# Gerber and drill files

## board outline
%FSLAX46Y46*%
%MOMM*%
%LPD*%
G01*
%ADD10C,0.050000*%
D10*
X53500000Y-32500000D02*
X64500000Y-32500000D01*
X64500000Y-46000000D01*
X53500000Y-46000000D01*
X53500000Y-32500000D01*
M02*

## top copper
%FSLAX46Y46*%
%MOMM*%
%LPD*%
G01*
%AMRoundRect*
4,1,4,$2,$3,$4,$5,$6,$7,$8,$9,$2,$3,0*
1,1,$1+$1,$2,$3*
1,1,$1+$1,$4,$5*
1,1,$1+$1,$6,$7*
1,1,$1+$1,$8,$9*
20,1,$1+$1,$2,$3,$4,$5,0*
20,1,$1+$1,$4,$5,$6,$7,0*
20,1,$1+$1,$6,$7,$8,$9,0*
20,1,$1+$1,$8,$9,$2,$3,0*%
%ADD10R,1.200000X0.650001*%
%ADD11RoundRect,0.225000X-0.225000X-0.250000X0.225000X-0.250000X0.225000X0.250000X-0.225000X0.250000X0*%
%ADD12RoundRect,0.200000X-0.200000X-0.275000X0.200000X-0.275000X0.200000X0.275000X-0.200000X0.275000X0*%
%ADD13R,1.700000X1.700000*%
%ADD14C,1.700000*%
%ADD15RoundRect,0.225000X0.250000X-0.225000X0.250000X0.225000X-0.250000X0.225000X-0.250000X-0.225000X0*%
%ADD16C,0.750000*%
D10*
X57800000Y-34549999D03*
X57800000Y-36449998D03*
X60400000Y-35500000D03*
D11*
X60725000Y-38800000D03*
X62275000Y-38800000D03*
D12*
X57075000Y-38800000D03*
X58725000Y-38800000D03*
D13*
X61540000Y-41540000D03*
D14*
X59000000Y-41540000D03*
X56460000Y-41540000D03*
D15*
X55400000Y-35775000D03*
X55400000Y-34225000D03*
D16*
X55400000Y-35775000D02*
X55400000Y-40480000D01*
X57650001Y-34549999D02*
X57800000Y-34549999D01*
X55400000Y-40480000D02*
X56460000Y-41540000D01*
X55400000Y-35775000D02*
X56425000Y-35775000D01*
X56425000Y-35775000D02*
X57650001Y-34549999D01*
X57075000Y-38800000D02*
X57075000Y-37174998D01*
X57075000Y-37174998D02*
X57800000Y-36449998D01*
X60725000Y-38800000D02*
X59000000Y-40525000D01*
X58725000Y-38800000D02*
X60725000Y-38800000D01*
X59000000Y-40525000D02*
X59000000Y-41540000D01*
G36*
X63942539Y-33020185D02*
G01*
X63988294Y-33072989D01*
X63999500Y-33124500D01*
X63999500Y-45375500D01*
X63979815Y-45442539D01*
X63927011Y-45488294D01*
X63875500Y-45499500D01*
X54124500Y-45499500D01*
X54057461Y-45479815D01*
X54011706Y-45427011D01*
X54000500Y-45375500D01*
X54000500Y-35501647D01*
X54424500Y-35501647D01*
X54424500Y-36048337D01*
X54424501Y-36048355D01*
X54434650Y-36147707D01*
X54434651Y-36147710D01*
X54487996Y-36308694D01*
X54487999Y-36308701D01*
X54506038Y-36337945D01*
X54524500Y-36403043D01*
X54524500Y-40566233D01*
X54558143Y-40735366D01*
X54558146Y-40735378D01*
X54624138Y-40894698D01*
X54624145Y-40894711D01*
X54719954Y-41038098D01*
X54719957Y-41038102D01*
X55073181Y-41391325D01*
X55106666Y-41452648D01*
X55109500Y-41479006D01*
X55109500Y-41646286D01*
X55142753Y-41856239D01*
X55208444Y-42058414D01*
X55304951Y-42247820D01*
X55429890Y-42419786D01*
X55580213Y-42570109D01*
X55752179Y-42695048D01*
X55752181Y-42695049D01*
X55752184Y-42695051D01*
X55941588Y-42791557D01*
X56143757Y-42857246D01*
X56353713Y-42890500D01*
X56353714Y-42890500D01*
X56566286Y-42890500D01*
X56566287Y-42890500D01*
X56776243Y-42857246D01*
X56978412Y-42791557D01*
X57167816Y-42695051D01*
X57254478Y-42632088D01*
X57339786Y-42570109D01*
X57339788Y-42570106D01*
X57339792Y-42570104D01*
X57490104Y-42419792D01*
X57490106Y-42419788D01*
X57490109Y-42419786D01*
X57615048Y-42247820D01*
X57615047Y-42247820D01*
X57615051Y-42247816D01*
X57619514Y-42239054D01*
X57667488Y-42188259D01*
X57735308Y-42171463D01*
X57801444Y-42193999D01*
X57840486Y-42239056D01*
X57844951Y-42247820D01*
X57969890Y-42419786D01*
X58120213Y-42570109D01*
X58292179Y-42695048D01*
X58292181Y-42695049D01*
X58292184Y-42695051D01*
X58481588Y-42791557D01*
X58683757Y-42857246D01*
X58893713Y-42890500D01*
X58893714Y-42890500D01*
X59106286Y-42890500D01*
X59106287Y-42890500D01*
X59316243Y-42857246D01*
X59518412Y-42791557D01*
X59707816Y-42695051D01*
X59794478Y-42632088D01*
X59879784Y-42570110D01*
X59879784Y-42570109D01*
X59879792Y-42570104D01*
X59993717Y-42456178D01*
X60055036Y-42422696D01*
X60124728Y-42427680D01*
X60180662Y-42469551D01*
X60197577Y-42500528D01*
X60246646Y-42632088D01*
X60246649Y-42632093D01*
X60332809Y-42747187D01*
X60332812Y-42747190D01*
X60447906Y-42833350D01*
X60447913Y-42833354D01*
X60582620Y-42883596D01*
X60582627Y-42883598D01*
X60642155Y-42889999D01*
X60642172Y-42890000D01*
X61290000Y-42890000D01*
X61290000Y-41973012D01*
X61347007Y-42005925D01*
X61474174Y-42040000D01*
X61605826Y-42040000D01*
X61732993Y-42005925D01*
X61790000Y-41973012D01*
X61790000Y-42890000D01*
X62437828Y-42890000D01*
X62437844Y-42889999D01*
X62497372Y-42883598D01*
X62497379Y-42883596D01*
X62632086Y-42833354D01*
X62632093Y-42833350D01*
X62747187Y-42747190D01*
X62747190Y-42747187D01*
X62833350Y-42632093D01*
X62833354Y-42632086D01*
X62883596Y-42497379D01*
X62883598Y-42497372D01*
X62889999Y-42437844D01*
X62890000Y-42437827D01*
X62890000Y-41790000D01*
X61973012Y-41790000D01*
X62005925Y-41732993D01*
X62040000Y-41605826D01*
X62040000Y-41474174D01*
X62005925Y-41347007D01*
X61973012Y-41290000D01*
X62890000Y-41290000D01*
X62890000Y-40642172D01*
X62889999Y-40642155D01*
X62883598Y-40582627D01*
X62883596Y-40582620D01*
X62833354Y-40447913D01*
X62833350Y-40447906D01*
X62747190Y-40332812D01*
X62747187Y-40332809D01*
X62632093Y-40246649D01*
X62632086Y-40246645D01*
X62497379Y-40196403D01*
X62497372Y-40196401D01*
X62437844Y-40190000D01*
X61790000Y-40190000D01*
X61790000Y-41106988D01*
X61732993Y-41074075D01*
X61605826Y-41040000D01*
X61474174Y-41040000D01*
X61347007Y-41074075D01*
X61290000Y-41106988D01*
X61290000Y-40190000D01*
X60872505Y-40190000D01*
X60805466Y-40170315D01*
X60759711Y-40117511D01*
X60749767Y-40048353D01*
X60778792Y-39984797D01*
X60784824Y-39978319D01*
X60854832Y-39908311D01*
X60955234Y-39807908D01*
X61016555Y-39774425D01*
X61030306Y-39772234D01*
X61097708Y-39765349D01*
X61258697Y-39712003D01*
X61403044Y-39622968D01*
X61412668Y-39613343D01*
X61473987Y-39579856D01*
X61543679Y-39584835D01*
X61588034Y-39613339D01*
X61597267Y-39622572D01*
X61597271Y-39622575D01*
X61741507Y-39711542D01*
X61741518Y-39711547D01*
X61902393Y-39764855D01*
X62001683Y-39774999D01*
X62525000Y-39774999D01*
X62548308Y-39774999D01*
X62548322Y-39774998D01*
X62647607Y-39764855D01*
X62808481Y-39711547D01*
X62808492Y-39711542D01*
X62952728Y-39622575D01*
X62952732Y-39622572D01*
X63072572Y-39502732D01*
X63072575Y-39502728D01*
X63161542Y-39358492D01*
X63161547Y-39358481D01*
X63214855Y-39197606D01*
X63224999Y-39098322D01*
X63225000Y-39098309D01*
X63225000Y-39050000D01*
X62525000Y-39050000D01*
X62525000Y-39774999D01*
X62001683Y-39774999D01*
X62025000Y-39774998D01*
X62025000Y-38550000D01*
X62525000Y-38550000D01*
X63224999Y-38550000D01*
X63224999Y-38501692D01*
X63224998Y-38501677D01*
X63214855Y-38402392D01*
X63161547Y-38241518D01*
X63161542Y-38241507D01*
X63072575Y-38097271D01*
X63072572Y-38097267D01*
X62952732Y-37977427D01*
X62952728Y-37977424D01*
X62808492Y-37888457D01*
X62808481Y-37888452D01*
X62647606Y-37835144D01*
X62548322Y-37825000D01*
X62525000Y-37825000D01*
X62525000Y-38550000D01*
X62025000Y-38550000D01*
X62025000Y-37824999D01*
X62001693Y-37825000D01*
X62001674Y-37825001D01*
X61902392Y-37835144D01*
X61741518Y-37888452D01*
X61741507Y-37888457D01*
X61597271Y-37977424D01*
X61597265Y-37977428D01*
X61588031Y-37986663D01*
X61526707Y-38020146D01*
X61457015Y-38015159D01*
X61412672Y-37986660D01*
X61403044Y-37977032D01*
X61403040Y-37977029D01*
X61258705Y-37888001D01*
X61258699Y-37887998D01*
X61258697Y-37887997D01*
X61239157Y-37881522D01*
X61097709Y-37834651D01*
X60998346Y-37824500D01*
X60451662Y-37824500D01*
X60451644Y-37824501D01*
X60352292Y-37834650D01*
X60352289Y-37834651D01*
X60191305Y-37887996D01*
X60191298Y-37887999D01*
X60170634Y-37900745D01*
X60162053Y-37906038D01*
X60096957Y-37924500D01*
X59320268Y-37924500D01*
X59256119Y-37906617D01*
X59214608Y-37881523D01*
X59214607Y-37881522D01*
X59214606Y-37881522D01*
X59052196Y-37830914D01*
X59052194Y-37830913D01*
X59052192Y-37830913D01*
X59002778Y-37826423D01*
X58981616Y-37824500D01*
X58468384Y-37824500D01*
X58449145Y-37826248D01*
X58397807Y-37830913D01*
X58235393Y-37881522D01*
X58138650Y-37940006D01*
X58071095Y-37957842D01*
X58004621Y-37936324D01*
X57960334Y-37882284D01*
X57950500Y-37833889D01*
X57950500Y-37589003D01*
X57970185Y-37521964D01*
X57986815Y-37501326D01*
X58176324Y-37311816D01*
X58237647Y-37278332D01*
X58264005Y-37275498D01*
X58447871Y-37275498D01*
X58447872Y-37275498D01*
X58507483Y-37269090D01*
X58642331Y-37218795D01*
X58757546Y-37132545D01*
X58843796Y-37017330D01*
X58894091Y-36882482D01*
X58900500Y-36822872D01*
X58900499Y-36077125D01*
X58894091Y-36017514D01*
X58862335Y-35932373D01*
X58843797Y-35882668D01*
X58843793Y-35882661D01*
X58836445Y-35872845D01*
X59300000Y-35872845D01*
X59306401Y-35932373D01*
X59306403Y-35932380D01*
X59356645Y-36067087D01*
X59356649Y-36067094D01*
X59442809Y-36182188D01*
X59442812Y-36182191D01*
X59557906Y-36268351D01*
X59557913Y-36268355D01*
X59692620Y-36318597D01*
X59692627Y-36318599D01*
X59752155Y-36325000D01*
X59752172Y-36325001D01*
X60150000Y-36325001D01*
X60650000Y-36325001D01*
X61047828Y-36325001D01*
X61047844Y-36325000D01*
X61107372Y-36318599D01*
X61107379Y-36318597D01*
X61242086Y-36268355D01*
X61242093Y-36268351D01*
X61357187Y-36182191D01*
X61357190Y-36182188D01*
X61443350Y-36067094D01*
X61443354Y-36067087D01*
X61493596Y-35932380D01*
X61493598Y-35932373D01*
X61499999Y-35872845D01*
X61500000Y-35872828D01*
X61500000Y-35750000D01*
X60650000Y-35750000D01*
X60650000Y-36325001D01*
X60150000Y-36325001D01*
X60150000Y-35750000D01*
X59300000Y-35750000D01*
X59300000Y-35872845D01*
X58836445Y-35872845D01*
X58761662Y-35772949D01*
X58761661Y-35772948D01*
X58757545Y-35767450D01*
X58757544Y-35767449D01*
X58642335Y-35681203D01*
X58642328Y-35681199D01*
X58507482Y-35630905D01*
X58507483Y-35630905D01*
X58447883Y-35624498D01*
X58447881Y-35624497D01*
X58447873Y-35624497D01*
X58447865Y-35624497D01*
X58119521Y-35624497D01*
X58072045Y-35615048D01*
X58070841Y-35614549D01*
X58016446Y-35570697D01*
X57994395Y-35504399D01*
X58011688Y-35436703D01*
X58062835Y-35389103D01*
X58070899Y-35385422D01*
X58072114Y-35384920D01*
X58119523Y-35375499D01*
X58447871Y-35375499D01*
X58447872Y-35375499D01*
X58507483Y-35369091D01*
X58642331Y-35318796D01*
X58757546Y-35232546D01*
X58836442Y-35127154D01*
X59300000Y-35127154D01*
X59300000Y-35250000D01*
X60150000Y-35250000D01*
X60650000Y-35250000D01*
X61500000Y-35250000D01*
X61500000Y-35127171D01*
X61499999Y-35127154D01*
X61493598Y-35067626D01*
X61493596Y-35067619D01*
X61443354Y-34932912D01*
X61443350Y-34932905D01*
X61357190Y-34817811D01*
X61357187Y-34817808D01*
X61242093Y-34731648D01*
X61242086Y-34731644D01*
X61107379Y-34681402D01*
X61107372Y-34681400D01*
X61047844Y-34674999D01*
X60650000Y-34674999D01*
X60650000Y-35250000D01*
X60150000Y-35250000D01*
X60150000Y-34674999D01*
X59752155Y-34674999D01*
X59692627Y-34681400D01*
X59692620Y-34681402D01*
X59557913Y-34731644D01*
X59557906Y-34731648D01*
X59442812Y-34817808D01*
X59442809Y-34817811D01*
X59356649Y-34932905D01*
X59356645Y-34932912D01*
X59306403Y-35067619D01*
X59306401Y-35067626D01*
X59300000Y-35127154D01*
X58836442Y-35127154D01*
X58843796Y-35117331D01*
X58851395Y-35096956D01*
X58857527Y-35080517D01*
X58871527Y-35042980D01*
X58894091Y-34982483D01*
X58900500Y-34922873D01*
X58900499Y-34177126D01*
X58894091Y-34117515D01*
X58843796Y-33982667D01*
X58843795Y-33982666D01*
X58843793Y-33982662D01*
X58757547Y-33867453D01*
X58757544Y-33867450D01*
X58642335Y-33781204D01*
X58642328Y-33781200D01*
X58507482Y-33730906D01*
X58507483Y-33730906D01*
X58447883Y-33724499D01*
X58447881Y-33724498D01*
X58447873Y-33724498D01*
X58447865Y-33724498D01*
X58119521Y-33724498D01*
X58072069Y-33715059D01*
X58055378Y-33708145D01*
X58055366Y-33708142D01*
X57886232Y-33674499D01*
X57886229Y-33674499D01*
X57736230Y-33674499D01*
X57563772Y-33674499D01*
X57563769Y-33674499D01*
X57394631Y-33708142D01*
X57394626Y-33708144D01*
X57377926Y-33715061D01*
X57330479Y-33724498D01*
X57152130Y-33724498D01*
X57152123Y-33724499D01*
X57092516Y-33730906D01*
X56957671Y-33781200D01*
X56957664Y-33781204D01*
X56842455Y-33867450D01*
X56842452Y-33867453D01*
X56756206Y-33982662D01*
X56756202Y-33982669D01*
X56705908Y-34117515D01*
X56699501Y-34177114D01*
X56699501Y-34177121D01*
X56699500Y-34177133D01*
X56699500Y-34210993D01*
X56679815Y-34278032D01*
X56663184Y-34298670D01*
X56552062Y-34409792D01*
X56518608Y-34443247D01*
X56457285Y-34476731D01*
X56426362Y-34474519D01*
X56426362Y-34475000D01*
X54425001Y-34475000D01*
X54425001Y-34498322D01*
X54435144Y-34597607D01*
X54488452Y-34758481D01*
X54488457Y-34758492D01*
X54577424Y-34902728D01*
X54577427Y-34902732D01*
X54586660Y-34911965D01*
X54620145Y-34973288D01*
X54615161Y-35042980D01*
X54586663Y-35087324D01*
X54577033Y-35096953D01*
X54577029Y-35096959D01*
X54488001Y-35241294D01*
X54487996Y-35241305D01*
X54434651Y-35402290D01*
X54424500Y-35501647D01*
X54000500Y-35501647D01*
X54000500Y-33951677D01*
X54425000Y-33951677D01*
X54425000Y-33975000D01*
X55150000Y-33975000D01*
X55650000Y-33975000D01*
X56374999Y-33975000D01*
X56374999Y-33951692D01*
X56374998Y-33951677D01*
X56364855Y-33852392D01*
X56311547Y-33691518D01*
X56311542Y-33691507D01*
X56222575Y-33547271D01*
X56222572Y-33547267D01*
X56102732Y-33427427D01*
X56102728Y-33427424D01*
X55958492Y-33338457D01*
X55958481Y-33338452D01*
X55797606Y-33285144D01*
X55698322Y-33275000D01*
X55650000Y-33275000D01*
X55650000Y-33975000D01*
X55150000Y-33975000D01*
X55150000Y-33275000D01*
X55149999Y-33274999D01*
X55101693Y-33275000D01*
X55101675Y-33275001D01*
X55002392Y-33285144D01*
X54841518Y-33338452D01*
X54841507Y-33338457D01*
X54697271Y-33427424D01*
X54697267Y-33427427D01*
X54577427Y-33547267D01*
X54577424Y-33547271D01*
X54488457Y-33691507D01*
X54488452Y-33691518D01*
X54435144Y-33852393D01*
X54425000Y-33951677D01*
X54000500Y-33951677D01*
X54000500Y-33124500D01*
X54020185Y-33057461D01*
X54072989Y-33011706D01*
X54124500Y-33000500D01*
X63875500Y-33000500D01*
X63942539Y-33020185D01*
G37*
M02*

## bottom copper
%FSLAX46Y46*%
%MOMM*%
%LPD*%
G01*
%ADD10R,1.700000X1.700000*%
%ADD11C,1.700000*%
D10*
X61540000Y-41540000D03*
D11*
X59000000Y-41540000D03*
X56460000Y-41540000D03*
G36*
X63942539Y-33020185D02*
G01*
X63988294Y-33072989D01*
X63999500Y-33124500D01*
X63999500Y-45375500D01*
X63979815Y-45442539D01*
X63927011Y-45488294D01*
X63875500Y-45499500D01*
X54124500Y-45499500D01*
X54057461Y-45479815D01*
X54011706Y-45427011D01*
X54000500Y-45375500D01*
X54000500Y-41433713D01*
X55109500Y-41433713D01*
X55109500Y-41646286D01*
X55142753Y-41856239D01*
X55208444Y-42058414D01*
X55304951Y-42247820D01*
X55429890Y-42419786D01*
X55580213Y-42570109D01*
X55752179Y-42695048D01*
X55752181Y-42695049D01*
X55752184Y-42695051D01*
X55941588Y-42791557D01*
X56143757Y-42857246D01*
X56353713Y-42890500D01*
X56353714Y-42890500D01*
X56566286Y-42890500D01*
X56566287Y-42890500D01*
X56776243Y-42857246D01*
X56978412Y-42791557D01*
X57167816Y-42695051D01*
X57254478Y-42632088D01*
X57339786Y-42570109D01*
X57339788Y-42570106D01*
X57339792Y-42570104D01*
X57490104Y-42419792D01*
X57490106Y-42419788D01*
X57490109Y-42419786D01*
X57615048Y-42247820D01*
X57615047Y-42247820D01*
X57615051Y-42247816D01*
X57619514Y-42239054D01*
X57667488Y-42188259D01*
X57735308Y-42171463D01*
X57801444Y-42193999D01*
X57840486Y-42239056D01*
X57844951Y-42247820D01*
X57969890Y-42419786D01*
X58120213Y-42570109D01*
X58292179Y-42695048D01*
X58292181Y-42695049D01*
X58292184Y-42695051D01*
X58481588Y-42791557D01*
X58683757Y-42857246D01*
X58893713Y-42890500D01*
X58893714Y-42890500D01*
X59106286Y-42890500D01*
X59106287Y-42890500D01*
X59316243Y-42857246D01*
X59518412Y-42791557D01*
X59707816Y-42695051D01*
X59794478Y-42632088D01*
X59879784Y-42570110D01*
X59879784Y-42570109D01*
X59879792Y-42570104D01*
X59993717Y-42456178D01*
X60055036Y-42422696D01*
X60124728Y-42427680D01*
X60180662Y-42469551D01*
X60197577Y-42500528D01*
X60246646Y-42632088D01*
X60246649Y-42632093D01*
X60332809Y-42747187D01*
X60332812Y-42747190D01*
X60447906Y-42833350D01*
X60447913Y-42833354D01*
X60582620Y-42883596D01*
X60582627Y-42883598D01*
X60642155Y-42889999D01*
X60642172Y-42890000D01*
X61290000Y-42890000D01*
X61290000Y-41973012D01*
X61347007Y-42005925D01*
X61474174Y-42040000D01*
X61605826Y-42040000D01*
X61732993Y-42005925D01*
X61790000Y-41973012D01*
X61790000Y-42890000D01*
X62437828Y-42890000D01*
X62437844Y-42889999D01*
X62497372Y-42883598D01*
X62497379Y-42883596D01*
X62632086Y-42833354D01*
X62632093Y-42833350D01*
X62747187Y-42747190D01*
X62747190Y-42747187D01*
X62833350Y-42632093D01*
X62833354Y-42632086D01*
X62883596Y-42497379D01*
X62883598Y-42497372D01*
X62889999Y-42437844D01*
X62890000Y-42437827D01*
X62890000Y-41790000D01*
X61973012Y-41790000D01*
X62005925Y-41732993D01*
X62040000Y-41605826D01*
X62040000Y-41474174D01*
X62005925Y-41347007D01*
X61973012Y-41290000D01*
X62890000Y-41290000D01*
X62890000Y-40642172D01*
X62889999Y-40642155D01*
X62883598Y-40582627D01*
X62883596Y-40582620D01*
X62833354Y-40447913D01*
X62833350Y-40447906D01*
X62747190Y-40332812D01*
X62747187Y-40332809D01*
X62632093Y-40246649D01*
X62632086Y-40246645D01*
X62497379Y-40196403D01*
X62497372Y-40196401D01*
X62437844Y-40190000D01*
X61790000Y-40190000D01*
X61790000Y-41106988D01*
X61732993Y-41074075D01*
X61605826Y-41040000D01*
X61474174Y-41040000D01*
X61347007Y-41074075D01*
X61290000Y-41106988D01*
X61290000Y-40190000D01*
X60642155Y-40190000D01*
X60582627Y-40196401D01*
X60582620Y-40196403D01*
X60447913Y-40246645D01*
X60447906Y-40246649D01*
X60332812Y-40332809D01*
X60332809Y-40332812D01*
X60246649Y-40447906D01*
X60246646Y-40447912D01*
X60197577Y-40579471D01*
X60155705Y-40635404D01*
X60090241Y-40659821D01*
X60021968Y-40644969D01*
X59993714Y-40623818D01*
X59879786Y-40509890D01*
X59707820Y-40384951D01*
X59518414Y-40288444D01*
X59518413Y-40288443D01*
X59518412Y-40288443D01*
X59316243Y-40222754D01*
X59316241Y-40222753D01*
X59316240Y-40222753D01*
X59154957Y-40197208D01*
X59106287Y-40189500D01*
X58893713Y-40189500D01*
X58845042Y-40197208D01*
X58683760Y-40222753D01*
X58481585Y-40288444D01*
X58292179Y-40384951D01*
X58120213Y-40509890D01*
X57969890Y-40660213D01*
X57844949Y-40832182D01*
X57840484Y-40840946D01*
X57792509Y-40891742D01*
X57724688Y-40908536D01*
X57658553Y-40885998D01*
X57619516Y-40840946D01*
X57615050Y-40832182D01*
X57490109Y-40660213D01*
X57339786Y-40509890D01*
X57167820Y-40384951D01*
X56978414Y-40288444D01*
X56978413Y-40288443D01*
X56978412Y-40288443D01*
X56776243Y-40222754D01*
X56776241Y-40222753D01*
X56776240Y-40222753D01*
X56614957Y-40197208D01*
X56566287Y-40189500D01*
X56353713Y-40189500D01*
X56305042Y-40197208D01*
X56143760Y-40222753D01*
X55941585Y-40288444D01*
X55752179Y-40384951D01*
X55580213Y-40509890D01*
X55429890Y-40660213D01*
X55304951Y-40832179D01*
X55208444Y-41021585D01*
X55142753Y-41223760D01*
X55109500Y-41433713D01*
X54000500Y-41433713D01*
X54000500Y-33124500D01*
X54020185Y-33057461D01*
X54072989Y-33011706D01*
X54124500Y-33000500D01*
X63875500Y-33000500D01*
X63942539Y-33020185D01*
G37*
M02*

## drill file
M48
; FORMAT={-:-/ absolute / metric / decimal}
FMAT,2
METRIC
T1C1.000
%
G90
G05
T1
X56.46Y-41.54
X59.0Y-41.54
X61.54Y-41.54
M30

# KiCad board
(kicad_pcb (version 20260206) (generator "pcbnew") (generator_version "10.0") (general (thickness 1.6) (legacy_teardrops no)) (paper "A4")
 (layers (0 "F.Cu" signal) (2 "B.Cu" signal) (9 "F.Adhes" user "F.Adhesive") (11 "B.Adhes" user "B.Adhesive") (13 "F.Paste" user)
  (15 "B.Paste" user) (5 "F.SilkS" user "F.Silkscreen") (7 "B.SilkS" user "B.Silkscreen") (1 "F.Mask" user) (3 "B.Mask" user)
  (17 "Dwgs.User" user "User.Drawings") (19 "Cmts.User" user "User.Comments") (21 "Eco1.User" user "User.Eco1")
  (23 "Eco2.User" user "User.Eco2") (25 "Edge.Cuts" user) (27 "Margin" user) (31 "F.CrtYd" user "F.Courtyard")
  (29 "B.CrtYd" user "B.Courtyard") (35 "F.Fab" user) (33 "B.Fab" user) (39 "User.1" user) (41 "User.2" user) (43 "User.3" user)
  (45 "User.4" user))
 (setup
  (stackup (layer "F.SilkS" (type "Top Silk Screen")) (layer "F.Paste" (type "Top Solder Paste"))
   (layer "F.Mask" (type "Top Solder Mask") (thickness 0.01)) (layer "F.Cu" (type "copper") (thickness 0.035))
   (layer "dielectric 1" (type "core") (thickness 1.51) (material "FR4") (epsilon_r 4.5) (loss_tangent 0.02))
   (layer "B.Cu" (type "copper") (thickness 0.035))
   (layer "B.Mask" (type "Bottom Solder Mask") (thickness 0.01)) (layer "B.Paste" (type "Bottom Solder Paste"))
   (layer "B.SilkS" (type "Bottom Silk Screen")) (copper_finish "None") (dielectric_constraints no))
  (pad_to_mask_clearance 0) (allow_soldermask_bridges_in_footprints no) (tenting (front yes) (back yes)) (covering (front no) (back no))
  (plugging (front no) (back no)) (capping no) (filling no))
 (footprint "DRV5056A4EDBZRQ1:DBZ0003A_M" (layer "F.Cu") (at 59.1 35.5)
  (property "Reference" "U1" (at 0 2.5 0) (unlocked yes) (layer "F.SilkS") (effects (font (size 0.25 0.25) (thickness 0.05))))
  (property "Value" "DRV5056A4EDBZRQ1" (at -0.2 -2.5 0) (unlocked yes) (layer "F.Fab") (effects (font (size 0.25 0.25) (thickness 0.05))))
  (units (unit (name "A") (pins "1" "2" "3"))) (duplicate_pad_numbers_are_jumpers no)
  (pad "1" smd rect (at -1.3 -0.950001 90) (size 0.650001 1.2) (layers "F.Cu" "F.Mask" "F.Paste") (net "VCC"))
  (pad "2" smd rect (at -1.3 0.949998 90) (size 0.650001 1.2) (layers "F.Cu" "F.Mask" "F.Paste") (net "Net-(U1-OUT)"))
  (pad "3" smd rect (at 1.3 0 90) (size 0.650001 1.2) (layers "F.Cu" "F.Mask" "F.Paste") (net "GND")))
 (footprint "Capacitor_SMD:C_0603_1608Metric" (layer "F.Cu") (at 61.5 38.8)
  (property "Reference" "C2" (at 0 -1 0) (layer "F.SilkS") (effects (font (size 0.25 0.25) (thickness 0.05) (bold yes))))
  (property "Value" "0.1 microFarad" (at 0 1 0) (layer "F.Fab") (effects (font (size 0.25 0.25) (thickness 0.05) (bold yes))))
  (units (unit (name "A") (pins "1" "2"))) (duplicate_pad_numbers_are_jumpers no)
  (pad "1" smd roundrect (at -0.775 0) (size 0.9 0.95) (layers "F.Cu" "F.Mask" "F.Paste") (roundrect_rratio 0.25) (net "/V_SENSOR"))
  (pad "2" smd roundrect (at 0.775 0) (size 0.9 0.95) (layers "F.Cu" "F.Mask" "F.Paste") (roundrect_rratio 0.25) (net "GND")))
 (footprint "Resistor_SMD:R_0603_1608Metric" (layer "F.Cu") (at 57.9 38.8)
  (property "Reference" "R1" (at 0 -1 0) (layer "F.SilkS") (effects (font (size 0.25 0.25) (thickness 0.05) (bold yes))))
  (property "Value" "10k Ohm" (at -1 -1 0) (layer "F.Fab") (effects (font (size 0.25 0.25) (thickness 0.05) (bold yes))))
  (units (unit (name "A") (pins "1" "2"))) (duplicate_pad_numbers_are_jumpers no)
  (pad "1" smd roundrect (at -0.825 0) (size 0.8 0.95) (layers "F.Cu" "F.Mask" "F.Paste") (roundrect_rratio 0.25) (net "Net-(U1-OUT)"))
  (pad "2" smd roundrect (at 0.825 0) (size 0.8 0.95) (layers "F.Cu" "F.Mask" "F.Paste") (roundrect_rratio 0.25) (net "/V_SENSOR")))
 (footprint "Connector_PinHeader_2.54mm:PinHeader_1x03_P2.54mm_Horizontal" (layer "F.Cu") (at 61.54 41.54 -90)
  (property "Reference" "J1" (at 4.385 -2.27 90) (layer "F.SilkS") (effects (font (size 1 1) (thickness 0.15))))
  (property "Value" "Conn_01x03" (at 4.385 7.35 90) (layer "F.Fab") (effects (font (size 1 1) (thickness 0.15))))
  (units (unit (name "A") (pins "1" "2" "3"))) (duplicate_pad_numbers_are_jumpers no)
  (pad "1" thru_hole rect (at 0 0 270) (size 1.7 1.7) (drill 1) (layers "*.Cu" "*.Mask") (remove_unused_layers no) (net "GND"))
  (pad "2" thru_hole circle (at 0 2.54 270) (size 1.7 1.7) (drill 1) (layers "*.Cu" "*.Mask") (remove_unused_layers no) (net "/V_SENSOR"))
  (pad "3" thru_hole circle (at 0 5.08 270) (size 1.7 1.7) (drill 1) (layers "*.Cu" "*.Mask") (remove_unused_layers no) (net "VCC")))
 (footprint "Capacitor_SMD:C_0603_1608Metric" (layer "F.Cu") (at 55.4 35 90)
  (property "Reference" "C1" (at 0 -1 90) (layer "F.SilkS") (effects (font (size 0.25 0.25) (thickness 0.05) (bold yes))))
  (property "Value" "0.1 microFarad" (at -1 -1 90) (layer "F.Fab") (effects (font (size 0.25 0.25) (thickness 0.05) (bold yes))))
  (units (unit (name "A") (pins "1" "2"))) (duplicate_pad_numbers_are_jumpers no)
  (pad "1" smd roundrect (at -0.775 0 90) (size 0.9 0.95) (layers "F.Cu" "F.Mask" "F.Paste") (roundrect_rratio 0.25) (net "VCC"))
  (pad "2" smd roundrect (at 0.775 0 90) (size 0.9 0.95) (layers "F.Cu" "F.Mask" "F.Paste") (roundrect_rratio 0.25) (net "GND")))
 (gr_rect (start 53.5 32.5) (end 64.5 46) (stroke (width 0.05) (type solid)) (fill no) (layer "Edge.Cuts"))
 (segment (start 55.4 35.775) (end 55.4 40.48) (width 0.75) (layer "F.Cu") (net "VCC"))
 (segment (start 57.650001 34.549999) (end 57.8 34.549999) (width 0.75) (layer "F.Cu") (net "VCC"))
 (segment (start 55.4 40.48) (end 56.46 41.54) (width 0.75) (layer "F.Cu") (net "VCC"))
 (segment (start 55.4 35.775) (end 56.425 35.775) (width 0.75) (layer "F.Cu") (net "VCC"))
 (segment (start 56.425 35.775) (end 57.650001 34.549999) (width 0.75) (layer "F.Cu") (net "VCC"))
 (segment (start 57.075 38.8) (end 57.075 37.174998) (width 0.75) (layer "F.Cu") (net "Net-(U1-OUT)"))
 (segment (start 57.075 37.174998) (end 57.8 36.449998) (width 0.75) (layer "F.Cu") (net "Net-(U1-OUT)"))
 (segment (start 60.725 38.8) (end 59 40.525) (width 0.75) (layer "F.Cu") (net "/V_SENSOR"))
 (segment (start 58.725 38.8) (end 60.725 38.8) (width 0.75) (layer "F.Cu") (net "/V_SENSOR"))
 (segment (start 59 40.525) (end 59 41.54) (width 0.75) (layer "F.Cu") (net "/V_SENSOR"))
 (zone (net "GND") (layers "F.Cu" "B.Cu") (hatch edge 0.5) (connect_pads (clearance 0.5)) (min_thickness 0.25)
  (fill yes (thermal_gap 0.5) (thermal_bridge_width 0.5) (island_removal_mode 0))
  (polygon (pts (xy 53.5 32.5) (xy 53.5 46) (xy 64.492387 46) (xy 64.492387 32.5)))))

